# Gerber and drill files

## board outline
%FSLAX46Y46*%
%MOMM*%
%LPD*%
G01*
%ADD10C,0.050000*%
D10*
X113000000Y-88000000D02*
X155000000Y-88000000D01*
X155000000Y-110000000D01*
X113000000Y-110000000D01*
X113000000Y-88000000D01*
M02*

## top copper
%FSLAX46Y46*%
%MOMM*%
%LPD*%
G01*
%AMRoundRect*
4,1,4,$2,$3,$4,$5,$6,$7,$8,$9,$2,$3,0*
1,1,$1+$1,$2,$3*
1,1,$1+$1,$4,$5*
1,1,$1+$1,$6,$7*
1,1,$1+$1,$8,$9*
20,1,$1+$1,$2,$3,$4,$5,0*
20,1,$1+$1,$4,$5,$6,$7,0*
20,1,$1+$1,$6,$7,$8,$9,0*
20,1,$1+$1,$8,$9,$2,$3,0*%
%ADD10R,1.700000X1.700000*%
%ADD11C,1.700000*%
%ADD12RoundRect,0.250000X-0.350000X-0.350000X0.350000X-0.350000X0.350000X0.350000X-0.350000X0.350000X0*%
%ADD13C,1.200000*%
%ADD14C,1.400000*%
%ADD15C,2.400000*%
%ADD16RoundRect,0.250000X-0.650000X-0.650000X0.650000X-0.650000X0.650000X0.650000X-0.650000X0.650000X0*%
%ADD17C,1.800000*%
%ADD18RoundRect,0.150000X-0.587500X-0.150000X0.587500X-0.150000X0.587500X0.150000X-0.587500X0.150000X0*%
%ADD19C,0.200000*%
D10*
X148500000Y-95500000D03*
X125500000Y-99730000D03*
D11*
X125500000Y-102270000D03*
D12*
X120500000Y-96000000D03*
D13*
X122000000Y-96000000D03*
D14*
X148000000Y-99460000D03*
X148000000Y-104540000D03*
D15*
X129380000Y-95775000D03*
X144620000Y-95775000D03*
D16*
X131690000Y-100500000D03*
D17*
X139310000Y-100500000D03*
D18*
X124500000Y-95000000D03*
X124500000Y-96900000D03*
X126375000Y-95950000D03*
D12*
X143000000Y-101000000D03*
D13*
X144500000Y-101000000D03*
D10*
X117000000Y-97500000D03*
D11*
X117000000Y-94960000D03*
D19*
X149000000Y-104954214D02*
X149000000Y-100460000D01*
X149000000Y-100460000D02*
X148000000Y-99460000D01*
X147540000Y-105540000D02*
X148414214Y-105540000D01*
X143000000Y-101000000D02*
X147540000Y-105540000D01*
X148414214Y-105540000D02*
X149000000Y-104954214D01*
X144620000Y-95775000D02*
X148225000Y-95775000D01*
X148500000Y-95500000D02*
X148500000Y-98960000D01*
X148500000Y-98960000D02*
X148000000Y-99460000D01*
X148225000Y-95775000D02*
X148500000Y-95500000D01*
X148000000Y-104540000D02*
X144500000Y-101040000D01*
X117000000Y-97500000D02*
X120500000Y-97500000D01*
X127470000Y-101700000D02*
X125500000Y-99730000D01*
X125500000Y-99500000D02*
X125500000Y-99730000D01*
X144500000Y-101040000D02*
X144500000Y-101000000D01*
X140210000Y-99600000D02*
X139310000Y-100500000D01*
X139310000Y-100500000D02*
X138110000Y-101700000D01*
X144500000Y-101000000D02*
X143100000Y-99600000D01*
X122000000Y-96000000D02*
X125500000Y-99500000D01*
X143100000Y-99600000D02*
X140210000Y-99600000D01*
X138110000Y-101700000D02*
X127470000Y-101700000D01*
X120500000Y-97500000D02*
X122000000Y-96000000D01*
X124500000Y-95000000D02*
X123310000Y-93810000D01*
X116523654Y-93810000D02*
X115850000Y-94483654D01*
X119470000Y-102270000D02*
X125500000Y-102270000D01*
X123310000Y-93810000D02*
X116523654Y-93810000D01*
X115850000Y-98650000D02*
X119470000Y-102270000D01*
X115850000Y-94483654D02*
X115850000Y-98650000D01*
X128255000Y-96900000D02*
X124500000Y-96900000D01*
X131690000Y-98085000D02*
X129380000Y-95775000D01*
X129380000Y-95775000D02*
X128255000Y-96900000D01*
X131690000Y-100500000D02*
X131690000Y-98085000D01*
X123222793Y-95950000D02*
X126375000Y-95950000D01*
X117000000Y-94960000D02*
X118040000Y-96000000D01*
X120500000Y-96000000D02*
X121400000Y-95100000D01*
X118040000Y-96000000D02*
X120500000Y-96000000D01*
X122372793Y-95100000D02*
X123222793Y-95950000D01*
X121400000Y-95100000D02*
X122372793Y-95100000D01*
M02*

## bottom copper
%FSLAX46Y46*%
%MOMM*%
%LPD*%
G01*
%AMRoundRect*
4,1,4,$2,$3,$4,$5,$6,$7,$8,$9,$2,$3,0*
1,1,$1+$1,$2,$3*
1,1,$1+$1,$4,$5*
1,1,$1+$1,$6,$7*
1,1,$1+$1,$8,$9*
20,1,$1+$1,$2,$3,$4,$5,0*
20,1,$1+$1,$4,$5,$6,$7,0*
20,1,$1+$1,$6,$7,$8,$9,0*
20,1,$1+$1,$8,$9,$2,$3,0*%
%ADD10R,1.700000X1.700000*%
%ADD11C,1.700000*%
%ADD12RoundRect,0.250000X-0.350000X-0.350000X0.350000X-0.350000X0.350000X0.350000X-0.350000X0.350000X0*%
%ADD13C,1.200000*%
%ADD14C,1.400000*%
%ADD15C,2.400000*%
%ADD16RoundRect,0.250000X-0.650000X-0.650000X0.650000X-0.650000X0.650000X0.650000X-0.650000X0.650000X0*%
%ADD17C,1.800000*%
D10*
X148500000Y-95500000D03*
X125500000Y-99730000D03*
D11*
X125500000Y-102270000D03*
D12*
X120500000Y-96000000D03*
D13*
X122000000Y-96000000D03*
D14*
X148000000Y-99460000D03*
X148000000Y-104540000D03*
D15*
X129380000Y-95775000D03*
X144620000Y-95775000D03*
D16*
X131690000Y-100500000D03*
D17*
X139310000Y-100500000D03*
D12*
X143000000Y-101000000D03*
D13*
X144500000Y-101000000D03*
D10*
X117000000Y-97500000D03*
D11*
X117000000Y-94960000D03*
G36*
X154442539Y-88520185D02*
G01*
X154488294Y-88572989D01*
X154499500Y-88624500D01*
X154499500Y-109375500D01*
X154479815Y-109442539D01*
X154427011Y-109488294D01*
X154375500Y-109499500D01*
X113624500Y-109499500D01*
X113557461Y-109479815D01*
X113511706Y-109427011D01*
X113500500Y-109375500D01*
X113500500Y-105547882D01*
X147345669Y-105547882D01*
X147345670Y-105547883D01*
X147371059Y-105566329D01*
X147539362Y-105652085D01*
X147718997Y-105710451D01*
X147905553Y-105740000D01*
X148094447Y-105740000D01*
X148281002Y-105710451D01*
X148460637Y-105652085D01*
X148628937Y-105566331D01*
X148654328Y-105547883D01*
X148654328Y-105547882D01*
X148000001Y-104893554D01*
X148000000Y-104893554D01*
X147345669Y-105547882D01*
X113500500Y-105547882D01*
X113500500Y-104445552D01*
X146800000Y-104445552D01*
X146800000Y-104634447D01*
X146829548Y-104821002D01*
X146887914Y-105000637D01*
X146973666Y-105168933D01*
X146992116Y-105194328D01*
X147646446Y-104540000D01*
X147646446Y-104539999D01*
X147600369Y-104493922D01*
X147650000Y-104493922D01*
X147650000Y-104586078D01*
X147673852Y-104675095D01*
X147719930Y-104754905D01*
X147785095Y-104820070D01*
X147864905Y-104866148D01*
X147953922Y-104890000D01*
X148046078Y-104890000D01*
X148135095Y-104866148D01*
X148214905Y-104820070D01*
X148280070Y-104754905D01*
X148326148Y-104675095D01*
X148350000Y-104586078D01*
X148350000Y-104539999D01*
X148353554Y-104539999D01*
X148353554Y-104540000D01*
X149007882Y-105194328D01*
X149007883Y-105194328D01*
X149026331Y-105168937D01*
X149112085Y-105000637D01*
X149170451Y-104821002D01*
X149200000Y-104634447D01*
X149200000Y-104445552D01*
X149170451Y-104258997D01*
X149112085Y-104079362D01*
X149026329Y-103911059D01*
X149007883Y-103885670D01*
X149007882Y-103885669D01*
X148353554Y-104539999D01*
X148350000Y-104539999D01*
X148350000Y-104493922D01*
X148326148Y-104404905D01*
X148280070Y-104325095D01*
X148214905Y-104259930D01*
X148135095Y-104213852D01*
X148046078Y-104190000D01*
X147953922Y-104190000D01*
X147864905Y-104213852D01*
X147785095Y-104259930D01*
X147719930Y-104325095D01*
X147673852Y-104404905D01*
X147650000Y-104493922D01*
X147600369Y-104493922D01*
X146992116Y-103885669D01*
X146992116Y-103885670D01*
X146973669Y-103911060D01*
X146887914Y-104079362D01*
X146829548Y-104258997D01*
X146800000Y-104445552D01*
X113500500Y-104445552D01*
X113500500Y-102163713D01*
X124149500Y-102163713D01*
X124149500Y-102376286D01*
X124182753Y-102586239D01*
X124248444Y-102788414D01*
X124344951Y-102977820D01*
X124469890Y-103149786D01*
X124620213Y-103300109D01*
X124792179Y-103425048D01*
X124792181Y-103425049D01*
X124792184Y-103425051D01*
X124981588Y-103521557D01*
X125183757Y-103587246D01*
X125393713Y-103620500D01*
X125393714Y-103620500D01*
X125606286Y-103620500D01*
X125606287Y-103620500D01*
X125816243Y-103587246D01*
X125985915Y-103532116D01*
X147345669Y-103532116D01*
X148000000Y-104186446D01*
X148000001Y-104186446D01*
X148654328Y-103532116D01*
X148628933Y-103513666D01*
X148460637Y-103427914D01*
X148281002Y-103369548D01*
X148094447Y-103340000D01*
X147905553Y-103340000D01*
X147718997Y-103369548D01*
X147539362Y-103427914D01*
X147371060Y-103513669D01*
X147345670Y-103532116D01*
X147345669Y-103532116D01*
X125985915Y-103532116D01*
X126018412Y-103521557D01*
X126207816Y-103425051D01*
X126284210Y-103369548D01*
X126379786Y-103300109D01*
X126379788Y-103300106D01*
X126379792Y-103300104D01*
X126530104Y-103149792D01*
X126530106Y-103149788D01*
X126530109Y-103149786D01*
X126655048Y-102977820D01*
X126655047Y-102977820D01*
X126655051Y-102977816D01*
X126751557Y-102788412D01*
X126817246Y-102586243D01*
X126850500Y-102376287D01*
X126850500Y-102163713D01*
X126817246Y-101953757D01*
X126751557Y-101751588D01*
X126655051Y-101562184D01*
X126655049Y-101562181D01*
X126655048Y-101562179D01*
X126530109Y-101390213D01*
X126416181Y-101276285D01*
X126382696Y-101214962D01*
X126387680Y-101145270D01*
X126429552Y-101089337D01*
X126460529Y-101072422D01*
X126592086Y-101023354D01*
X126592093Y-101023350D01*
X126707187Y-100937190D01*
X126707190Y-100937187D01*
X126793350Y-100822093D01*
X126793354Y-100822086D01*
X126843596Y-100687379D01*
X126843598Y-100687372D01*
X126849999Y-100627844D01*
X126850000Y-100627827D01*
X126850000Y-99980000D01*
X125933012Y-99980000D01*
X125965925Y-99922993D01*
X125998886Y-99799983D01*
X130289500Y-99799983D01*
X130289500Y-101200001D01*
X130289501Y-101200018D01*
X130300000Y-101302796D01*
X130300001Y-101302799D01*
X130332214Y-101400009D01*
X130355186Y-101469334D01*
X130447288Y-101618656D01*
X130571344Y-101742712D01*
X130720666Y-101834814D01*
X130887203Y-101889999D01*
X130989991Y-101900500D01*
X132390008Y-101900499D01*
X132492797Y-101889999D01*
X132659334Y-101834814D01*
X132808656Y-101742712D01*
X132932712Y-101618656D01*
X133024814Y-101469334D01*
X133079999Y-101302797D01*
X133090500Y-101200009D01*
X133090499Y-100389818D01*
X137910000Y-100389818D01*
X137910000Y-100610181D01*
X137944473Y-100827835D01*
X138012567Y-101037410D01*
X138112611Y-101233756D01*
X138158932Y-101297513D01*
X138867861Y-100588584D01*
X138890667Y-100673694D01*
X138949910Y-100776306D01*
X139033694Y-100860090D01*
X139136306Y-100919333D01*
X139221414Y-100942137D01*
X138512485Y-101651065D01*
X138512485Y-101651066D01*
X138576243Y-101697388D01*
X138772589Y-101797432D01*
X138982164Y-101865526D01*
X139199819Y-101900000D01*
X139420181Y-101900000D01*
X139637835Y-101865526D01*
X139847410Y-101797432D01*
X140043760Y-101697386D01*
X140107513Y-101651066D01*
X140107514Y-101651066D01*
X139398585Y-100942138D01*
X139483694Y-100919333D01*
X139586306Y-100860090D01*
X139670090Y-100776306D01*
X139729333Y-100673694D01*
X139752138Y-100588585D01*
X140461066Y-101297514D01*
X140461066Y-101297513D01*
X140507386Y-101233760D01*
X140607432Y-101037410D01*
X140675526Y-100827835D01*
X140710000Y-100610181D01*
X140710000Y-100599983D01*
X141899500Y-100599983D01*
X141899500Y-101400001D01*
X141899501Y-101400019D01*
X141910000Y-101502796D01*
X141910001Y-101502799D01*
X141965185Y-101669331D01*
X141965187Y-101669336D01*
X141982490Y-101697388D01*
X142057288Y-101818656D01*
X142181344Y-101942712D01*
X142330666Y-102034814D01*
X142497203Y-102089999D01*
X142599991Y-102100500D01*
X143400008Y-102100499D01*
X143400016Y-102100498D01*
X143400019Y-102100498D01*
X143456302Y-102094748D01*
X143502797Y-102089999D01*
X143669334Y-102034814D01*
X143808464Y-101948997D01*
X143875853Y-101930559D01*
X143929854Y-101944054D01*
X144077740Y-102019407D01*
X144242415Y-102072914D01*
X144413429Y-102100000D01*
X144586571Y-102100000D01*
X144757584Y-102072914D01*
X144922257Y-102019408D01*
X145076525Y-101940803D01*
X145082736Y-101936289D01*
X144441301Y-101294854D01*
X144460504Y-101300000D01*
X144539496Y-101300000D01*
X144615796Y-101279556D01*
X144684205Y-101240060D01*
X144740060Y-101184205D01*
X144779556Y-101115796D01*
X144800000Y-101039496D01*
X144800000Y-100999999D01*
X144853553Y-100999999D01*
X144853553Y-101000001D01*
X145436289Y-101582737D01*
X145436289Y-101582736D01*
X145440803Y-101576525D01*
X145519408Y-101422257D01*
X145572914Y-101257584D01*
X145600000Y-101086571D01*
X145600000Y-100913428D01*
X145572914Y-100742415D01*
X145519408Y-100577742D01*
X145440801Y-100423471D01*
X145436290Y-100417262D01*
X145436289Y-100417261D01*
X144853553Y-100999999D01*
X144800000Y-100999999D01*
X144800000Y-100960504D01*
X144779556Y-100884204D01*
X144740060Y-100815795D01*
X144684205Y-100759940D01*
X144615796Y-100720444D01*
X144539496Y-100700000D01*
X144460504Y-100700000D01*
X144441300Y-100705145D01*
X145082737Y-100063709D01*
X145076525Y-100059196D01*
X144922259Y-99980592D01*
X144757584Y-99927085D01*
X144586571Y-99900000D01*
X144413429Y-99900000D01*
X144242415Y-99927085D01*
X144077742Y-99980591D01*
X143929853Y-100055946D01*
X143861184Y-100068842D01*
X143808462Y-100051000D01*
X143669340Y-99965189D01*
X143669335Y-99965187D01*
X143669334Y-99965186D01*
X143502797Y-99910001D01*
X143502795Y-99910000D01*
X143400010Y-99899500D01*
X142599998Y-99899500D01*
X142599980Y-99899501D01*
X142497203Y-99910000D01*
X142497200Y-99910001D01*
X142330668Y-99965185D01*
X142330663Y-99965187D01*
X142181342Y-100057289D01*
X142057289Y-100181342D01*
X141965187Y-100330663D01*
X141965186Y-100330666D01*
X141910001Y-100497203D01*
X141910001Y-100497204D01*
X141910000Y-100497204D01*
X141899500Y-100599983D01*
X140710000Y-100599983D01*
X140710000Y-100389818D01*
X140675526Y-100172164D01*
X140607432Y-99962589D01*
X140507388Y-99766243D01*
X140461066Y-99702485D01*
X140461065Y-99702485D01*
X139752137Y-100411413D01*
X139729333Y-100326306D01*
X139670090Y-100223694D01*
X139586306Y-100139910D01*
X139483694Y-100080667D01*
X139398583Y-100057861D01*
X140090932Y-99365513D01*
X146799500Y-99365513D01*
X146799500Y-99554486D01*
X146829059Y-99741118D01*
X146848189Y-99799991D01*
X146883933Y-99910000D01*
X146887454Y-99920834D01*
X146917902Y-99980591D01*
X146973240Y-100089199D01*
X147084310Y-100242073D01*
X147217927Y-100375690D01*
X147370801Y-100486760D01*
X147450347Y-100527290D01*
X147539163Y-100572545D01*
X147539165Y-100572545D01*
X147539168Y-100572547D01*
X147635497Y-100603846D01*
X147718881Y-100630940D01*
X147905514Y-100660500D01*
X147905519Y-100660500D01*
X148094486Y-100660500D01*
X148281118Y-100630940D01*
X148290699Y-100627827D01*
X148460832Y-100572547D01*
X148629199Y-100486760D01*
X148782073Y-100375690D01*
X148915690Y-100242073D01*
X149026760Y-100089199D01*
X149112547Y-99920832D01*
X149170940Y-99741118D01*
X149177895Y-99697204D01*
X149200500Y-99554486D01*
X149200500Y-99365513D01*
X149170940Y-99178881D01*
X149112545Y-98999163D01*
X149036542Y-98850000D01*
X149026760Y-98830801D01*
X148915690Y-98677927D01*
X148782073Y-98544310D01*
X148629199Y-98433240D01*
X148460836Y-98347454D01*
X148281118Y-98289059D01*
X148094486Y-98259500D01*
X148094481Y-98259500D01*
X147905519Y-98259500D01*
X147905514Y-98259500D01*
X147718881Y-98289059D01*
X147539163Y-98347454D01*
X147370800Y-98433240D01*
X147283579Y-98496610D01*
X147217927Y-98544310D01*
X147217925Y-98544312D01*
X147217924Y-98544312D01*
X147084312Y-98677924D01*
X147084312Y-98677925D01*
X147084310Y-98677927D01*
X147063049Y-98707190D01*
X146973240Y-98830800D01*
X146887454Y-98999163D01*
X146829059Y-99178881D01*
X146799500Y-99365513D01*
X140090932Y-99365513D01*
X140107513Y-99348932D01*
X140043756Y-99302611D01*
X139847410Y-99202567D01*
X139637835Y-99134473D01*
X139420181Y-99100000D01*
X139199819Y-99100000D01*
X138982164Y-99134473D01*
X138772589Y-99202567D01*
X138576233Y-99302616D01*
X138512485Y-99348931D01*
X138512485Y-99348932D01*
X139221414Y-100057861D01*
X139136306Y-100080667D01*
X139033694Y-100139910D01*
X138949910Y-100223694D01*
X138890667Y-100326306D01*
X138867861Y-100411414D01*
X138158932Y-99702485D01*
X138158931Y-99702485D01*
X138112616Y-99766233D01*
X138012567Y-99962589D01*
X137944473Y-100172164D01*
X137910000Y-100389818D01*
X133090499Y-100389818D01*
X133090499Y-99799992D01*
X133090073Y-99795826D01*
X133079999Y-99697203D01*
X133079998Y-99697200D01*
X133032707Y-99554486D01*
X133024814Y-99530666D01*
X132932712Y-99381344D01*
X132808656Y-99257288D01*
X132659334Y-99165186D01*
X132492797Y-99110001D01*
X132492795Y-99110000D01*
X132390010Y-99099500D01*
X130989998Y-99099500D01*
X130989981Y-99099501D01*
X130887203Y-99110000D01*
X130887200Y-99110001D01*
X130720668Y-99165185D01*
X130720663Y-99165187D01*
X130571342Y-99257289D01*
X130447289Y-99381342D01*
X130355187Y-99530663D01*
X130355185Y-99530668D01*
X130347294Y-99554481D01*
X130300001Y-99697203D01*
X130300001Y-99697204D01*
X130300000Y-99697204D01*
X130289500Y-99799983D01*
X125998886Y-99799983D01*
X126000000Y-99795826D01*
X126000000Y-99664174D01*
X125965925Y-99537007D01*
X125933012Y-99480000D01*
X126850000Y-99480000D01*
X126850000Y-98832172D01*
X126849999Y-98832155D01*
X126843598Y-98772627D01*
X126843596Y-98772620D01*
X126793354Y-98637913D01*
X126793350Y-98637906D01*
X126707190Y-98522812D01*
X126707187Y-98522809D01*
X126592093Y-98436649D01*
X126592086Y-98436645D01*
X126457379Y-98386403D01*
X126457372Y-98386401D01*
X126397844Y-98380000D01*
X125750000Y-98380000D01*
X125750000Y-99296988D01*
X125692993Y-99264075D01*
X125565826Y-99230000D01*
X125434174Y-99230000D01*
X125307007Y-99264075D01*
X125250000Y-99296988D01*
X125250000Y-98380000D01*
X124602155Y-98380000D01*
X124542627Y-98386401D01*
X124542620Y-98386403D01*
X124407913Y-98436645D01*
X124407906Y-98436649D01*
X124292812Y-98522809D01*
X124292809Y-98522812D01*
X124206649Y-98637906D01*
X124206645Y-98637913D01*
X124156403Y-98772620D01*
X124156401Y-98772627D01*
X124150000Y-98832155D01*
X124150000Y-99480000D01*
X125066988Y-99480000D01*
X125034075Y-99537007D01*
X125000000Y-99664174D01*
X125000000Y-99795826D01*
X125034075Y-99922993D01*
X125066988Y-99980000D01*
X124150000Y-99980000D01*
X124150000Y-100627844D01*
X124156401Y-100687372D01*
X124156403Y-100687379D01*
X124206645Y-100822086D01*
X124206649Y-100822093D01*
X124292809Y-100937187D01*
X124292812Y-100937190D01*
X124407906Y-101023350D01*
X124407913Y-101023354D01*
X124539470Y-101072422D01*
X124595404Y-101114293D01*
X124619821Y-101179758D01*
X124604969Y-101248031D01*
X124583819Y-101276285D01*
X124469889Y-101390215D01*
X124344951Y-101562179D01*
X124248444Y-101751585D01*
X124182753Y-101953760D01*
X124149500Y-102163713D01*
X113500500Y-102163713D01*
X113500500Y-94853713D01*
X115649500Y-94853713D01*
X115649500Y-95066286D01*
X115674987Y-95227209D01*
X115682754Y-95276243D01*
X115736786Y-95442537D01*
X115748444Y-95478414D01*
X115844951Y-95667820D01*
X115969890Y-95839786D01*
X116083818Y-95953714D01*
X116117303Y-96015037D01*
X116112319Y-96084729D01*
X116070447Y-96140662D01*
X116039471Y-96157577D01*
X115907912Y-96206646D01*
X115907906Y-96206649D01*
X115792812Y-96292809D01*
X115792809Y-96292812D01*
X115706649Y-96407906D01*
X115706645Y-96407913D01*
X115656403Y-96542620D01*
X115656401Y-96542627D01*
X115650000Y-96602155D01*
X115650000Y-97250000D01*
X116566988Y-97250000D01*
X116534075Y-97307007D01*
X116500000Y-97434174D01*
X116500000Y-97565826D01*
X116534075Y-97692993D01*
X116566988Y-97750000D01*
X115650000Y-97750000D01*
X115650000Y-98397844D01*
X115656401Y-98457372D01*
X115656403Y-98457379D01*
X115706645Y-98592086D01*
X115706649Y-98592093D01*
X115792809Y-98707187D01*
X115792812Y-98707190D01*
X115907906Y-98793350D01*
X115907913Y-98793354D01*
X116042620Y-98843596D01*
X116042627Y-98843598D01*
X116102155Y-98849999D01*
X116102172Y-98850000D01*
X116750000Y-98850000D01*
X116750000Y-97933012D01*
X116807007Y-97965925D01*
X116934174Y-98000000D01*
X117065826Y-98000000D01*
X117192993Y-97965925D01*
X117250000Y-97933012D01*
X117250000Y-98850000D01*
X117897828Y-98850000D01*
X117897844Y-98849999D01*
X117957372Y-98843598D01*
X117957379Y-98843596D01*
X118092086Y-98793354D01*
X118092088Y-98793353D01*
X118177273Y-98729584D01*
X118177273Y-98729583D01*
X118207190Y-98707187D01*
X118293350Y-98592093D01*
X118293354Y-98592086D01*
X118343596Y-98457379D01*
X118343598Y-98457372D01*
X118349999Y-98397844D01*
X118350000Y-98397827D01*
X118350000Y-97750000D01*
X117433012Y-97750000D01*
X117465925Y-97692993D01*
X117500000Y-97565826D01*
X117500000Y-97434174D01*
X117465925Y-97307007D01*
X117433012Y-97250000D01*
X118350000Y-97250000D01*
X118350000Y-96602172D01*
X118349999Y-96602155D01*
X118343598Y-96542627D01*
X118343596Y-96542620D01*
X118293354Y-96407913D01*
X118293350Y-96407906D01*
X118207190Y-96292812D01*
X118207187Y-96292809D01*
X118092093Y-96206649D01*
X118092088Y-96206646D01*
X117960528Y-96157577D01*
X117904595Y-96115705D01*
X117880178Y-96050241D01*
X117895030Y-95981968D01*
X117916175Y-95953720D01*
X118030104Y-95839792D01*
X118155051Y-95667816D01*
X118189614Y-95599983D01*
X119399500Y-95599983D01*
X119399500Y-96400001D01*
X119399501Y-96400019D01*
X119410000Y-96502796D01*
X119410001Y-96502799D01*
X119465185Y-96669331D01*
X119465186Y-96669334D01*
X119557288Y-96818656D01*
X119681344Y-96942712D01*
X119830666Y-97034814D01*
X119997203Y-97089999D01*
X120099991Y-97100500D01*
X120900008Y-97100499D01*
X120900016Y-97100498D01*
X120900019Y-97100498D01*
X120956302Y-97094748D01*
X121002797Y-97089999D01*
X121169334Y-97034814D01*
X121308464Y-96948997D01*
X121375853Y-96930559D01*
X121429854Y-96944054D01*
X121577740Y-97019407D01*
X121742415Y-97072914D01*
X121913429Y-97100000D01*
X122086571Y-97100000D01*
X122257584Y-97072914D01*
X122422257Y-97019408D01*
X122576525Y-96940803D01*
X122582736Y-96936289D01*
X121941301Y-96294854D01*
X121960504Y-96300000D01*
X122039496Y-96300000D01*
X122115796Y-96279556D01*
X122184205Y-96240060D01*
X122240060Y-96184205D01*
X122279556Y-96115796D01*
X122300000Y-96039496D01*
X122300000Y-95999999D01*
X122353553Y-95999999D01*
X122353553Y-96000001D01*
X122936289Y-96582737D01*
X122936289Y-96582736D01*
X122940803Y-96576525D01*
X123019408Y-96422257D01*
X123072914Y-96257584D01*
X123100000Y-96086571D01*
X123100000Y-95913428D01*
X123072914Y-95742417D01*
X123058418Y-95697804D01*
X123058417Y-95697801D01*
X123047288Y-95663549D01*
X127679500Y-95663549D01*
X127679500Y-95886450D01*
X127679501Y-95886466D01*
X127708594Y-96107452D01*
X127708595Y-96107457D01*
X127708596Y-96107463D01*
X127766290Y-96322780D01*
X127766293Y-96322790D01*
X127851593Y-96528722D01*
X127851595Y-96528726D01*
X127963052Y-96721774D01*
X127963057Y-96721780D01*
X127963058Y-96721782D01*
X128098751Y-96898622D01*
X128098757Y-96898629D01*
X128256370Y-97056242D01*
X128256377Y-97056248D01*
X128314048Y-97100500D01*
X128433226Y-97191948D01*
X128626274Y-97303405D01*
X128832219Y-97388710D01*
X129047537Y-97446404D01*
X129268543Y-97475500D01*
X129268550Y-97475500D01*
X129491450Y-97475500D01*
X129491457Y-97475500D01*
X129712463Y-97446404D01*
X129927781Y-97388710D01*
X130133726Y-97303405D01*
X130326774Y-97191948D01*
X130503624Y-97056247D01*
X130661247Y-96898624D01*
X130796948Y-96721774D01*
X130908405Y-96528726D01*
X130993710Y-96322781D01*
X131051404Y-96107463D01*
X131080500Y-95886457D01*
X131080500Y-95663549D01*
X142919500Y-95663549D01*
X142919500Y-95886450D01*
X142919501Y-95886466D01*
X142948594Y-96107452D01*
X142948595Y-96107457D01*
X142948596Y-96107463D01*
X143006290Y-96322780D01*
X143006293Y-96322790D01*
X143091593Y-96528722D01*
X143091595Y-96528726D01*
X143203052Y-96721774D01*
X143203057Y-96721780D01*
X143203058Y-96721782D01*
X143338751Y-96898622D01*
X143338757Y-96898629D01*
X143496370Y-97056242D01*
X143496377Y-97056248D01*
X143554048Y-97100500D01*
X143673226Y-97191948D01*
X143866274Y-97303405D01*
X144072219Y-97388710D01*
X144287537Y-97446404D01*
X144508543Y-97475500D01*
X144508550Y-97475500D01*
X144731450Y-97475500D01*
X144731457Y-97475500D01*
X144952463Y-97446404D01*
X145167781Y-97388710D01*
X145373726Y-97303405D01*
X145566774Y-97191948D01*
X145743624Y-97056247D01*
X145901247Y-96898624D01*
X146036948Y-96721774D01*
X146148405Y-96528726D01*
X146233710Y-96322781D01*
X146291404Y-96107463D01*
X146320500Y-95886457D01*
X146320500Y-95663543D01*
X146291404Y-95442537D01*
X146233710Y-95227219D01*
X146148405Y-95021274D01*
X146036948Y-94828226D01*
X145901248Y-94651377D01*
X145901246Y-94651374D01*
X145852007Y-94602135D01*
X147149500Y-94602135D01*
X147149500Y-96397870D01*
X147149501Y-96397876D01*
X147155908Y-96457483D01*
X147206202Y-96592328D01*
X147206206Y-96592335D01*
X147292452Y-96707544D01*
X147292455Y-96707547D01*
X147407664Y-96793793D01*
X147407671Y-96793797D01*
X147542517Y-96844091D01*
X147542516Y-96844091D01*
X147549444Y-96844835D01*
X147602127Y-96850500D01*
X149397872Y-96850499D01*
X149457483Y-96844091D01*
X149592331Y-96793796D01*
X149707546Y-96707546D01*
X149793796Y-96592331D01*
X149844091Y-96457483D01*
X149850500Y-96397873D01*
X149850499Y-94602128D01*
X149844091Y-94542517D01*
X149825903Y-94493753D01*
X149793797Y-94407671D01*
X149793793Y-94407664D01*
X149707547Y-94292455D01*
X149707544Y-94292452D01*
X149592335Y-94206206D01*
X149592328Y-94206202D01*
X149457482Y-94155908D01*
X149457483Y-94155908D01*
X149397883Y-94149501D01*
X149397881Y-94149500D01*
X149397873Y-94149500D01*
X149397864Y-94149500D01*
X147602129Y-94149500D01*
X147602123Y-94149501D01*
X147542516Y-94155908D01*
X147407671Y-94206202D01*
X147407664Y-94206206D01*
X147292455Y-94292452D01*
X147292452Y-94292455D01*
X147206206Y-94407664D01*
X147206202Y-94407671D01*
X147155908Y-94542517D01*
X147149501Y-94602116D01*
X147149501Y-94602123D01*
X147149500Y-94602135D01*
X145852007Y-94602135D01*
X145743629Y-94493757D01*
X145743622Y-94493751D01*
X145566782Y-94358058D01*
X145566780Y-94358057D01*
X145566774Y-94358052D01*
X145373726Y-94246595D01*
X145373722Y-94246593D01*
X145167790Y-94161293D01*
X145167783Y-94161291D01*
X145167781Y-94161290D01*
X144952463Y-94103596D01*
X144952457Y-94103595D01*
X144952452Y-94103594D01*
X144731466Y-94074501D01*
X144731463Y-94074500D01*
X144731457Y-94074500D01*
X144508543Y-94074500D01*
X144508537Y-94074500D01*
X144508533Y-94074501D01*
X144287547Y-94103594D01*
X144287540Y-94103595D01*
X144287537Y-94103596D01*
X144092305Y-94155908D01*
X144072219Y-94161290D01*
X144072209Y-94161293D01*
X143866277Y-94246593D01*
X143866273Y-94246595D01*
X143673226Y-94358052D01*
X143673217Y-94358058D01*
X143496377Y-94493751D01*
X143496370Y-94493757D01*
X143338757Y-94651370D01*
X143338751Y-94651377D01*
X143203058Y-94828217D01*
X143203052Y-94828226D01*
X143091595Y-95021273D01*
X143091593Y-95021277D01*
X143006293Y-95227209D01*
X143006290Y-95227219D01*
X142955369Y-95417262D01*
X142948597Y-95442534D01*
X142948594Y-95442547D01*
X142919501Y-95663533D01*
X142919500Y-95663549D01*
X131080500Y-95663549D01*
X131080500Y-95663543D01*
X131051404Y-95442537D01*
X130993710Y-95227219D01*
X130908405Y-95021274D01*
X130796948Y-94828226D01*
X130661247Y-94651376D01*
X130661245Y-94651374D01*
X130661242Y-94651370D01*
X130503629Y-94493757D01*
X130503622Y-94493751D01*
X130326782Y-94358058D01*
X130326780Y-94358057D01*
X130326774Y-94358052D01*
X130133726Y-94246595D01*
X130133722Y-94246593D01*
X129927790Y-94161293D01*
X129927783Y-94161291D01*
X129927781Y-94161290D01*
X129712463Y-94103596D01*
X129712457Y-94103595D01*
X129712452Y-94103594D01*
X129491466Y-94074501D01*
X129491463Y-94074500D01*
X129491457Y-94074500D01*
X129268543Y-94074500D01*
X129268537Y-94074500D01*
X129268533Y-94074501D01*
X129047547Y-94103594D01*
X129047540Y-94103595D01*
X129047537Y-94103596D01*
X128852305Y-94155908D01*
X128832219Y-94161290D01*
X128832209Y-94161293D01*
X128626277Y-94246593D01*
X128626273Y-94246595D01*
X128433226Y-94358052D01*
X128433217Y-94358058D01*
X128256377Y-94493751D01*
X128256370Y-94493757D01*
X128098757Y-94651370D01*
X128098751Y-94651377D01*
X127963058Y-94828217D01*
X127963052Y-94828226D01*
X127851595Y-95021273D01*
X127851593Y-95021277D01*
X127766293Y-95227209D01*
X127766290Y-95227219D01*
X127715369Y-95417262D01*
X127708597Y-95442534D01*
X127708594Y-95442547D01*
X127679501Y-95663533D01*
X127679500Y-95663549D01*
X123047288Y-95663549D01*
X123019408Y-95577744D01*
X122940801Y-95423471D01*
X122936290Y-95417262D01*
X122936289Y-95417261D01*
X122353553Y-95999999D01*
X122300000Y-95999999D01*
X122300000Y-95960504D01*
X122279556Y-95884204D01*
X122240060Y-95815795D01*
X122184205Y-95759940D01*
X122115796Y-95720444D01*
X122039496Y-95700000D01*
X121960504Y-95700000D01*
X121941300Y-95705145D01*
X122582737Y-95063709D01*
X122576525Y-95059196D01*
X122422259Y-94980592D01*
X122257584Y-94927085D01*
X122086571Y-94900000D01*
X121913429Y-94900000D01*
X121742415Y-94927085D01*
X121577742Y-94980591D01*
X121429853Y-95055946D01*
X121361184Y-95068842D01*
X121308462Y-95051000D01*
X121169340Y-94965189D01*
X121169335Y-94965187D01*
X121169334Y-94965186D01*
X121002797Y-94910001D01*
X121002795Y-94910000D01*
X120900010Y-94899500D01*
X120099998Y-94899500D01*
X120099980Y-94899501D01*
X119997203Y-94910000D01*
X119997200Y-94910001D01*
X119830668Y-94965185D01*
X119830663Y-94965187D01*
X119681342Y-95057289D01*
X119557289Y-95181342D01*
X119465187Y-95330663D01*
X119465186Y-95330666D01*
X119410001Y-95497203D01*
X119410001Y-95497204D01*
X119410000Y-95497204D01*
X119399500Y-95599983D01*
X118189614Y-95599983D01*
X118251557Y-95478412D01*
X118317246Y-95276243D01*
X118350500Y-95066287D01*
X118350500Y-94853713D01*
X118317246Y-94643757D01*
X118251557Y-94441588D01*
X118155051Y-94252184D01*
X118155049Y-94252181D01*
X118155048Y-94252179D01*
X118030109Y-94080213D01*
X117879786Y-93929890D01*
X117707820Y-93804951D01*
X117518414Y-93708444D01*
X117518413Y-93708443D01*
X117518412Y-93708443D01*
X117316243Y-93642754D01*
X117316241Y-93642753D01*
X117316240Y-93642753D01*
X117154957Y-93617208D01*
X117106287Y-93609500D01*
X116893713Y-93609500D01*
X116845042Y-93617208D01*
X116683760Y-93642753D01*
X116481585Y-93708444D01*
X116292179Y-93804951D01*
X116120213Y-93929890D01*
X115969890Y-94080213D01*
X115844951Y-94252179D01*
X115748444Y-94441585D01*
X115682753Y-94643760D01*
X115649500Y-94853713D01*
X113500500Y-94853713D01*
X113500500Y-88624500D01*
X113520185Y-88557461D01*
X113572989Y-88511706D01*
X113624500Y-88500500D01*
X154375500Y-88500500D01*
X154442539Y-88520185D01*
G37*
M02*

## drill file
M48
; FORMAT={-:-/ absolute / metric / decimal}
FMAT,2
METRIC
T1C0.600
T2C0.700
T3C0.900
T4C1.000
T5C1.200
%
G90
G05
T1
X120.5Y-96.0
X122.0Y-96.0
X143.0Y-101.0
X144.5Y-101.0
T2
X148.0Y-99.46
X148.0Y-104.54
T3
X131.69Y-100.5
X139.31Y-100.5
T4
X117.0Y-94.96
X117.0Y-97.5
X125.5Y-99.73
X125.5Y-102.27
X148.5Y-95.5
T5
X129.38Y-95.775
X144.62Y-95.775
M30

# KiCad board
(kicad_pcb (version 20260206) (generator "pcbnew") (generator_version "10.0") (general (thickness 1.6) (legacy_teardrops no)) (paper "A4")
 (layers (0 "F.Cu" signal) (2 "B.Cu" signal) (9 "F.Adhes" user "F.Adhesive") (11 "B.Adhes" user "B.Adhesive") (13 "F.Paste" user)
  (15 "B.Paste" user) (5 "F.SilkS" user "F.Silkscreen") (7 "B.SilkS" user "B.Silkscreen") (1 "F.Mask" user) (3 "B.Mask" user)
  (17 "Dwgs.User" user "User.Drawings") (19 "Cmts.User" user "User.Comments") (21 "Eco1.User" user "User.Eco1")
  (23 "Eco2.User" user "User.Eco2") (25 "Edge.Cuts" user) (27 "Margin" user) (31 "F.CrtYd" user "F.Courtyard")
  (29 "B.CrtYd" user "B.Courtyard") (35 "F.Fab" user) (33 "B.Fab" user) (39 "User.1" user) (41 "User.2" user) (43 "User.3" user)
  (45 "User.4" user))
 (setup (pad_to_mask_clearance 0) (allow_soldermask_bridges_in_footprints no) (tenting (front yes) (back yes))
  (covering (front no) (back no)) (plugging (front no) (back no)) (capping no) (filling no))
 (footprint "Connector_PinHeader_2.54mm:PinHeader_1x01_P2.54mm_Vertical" (layer "F.Cu") (at 148.5 95.5)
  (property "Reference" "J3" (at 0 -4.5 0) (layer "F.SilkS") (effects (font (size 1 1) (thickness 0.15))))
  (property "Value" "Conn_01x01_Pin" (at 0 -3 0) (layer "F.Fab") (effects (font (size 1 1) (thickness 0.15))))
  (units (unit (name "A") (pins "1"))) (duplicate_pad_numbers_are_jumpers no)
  (pad "1" thru_hole rect (at 0 0) (size 1.7 1.7) (drill 1) (layers "*.Cu" "*.Mask") (remove_unused_layers no) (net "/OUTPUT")))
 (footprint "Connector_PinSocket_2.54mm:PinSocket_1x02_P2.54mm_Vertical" (layer "F.Cu") (at 125.5 99.73)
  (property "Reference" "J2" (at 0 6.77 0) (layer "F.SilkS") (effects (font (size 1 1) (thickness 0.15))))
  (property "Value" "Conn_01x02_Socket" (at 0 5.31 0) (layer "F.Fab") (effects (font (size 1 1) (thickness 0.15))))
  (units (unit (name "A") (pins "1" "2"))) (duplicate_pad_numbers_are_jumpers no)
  (pad "1" thru_hole rect (at 0 0) (size 1.7 1.7) (drill 1) (layers "*.Cu" "*.Mask") (remove_unused_layers no) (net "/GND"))
  (pad "2" thru_hole circle (at 0 2.54) (size 1.7 1.7) (drill 1) (layers "*.Cu" "*.Mask") (remove_unused_layers no) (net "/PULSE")))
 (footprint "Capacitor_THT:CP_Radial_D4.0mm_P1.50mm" (layer "F.Cu") (at 120.5 96)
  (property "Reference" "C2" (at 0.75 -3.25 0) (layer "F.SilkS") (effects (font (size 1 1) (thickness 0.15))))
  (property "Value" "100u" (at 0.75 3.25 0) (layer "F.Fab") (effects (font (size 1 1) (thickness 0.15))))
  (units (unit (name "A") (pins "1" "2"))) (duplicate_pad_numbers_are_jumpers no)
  (pad "1" thru_hole roundrect (at 0 0) (size 1.2 1.2) (drill 0.6) (layers "*.Cu" "*.Mask") (remove_unused_layers no)
   (roundrect_rratio 0.208333) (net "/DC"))
  (pad "2" thru_hole circle (at 1.5 0) (size 1.2 1.2) (drill 0.6) (layers "*.Cu" "*.Mask") (remove_unused_layers no) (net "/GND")))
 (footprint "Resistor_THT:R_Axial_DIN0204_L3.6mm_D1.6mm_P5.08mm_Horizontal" (layer "F.Cu") (at 148 99.46 -90)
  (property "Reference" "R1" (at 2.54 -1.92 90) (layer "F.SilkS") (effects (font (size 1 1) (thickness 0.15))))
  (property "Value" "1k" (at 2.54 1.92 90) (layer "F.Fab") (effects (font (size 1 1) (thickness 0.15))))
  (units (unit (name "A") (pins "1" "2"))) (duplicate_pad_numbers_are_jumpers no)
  (pad "1" thru_hole circle (at 0 0 270) (size 1.4 1.4) (drill 0.7) (layers "*.Cu" "*.Mask") (remove_unused_layers no) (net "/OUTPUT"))
  (pad "2" thru_hole circle (at 5.08 0 270) (size 1.4 1.4) (drill 0.7) (layers "*.Cu" "*.Mask") (remove_unused_layers no) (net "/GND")))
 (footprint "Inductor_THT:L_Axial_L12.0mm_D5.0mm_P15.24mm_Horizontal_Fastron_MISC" (layer "F.Cu") (at 129.38 95.775)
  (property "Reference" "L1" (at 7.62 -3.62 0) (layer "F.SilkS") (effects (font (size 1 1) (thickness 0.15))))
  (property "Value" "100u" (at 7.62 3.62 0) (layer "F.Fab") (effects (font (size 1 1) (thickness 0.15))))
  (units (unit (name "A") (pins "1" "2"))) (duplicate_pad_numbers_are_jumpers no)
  (pad "1" thru_hole circle (at 0 0) (size 2.4 2.4) (drill 1.2) (layers "*.Cu" "*.Mask") (remove_unused_layers no) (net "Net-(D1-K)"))
  (pad "2" thru_hole circle (at 15.24 0) (size 2.4 2.4) (drill 1.2) (layers "*.Cu" "*.Mask") (remove_unused_layers no) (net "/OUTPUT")))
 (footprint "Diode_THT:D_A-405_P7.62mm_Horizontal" (layer "F.Cu") (at 131.69 100.5)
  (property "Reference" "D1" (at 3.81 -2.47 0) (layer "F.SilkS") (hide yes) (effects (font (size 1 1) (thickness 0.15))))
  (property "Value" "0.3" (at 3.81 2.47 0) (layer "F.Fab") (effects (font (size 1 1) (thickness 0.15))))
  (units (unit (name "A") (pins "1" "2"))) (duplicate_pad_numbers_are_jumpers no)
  (pad "1" thru_hole roundrect (at 0 0) (size 1.8 1.8) (drill 0.9) (layers "*.Cu" "*.Mask") (remove_unused_layers no)
   (roundrect_rratio 0.138889) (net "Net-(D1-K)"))
  (pad "2" thru_hole circle (at 7.62 0) (size 1.8 1.8) (drill 0.9) (layers "*.Cu" "*.Mask") (remove_unused_layers no) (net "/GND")))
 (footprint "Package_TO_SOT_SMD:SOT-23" (layer "F.Cu") (at 125.4375 95.95)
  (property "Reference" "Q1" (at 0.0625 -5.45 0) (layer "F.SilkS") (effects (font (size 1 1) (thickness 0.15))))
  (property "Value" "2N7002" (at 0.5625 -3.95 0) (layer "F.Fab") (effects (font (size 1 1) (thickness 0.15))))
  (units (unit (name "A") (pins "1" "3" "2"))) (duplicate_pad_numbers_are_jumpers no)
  (pad "1" smd roundrect (at -0.9375 -0.95) (size 1.475 0.6) (layers "F.Cu" "F.Mask" "F.Paste") (roundrect_rratio 0.25) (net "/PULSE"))
  (pad "2" smd roundrect (at -0.9375 0.95) (size 1.475 0.6) (layers "F.Cu" "F.Mask" "F.Paste") (roundrect_rratio 0.25) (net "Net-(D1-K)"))
  (pad "3" smd roundrect (at 0.9375 0) (size 1.475 0.6) (layers "F.Cu" "F.Mask" "F.Paste") (roundrect_rratio 0.25) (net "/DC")))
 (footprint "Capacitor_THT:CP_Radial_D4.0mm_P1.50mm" (layer "F.Cu") (at 143 101)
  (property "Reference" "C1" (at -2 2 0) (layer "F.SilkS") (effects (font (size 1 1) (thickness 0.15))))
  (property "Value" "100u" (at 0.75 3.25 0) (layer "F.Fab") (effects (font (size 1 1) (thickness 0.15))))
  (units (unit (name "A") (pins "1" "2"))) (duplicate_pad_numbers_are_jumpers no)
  (pad "1" thru_hole roundrect (at 0 0) (size 1.2 1.2) (drill 0.6) (layers "*.Cu" "*.Mask") (remove_unused_layers no)
   (roundrect_rratio 0.208333) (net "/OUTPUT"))
  (pad "2" thru_hole circle (at 1.5 0) (size 1.2 1.2) (drill 0.6) (layers "*.Cu" "*.Mask") (remove_unused_layers no) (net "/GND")))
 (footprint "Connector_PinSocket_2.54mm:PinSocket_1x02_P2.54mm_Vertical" (layer "F.Cu") (at 117 97.5 180)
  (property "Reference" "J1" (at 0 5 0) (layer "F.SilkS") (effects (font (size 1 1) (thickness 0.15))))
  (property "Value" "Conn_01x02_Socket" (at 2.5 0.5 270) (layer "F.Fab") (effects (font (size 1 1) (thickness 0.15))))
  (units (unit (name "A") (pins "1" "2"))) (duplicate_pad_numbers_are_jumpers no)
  (pad "1" thru_hole rect (at 0 0 180) (size 1.7 1.7) (drill 1) (layers "*.Cu" "*.Mask") (remove_unused_layers no) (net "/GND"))
  (pad "2" thru_hole circle (at 0 2.54 180) (size 1.7 1.7) (drill 1) (layers "*.Cu" "*.Mask") (remove_unused_layers no) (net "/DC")))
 (gr_rect (start 113 88) (end 155 110) (stroke (width 0.05) (type default)) (fill no) (layer "Edge.Cuts"))
 (segment (start 149 104.954214) (end 149 100.46) (width 0.2) (layer "F.Cu") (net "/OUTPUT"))
 (segment (start 149 100.46) (end 148 99.46) (width 0.2) (layer "F.Cu") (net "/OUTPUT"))
 (segment (start 147.54 105.54) (end 148.414214 105.54) (width 0.2) (layer "F.Cu") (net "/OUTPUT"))
 (segment (start 143 101) (end 147.54 105.54) (width 0.2) (layer "F.Cu") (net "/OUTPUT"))
 (segment (start 148.414214 105.54) (end 149 104.954214) (width 0.2) (layer "F.Cu") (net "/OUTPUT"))
 (segment (start 144.62 95.775) (end 148.225 95.775) (width 0.2) (layer "F.Cu") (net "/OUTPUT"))
 (segment (start 148.5 95.5) (end 148.5 98.96) (width 0.2) (layer "F.Cu") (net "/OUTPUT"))
 (segment (start 148.5 98.96) (end 148 99.46) (width 0.2) (layer "F.Cu") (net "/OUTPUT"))
 (segment (start 148.225 95.775) (end 148.5 95.5) (width 0.2) (layer "F.Cu") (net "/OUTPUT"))
 (segment (start 148 104.54) (end 144.5 101.04) (width 0.2) (layer "F.Cu") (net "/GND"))
 (segment (start 117 97.5) (end 120.5 97.5) (width 0.2) (layer "F.Cu") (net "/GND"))
 (segment (start 127.47 101.7) (end 125.5 99.73) (width 0.2) (layer "F.Cu") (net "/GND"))
 (segment (start 125.5 99.5) (end 125.5 99.73) (width 0.2) (layer "F.Cu") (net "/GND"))
 (segment (start 144.5 101.04) (end 144.5 101) (width 0.2) (layer "F.Cu") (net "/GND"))
 (segment (start 140.21 99.6) (end 139.31 100.5) (width 0.2) (layer "F.Cu") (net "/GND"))
 (segment (start 139.31 100.5) (end 138.11 101.7) (width 0.2) (layer "F.Cu") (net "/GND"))
 (segment (start 144.5 101) (end 143.1 99.6) (width 0.2) (layer "F.Cu") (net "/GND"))
 (segment (start 122 96) (end 125.5 99.5) (width 0.2) (layer "F.Cu") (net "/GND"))
 (segment (start 143.1 99.6) (end 140.21 99.6) (width 0.2) (layer "F.Cu") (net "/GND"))
 (segment (start 138.11 101.7) (end 127.47 101.7) (width 0.2) (layer "F.Cu") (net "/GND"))
 (segment (start 120.5 97.5) (end 122 96) (width 0.2) (layer "F.Cu") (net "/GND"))
 (segment (start 124.5 95) (end 123.31 93.81) (width 0.2) (layer "F.Cu") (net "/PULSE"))
 (segment (start 116.523654 93.81) (end 115.85 94.483654) (width 0.2) (layer "F.Cu") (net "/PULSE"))
 (segment (start 119.47 102.27) (end 125.5 102.27) (width 0.2) (layer "F.Cu") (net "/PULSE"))
 (segment (start 123.31 93.81) (end 116.523654 93.81) (width 0.2) (layer "F.Cu") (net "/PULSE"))
 (segment (start 115.85 98.65) (end 119.47 102.27) (width 0.2) (layer "F.Cu") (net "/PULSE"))
 (segment (start 115.85 94.483654) (end 115.85 98.65) (width 0.2) (layer "F.Cu") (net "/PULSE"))
 (segment (start 128.255 96.9) (end 124.5 96.9) (width 0.2) (layer "F.Cu") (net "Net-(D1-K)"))
 (segment (start 131.69 98.085) (end 129.38 95.775) (width 0.2) (layer "F.Cu") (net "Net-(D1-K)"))
 (segment (start 129.38 95.775) (end 128.255 96.9) (width 0.2) (layer "F.Cu") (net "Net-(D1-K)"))
 (segment (start 131.69 100.5) (end 131.69 98.085) (width 0.2) (layer "F.Cu") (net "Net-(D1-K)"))
 (segment (start 123.222793 95.95) (end 126.375 95.95) (width 0.2) (layer "F.Cu") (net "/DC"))
 (segment (start 117 94.96) (end 118.04 96) (width 0.2) (layer "F.Cu") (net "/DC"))
 (segment (start 120.5 96) (end 121.4 95.1) (width 0.2) (layer "F.Cu") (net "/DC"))
 (segment (start 118.04 96) (end 120.5 96) (width 0.2) (layer "F.Cu") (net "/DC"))
 (segment (start 122.372793 95.1) (end 123.222793 95.95) (width 0.2) (layer "F.Cu") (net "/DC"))
 (segment (start 121.4 95.1) (end 122.372793 95.1) (width 0.2) (layer "F.Cu") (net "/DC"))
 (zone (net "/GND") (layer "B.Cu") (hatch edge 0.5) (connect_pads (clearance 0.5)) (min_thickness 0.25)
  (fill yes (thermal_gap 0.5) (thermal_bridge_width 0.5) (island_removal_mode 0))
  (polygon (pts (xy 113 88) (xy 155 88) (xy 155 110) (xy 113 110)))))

